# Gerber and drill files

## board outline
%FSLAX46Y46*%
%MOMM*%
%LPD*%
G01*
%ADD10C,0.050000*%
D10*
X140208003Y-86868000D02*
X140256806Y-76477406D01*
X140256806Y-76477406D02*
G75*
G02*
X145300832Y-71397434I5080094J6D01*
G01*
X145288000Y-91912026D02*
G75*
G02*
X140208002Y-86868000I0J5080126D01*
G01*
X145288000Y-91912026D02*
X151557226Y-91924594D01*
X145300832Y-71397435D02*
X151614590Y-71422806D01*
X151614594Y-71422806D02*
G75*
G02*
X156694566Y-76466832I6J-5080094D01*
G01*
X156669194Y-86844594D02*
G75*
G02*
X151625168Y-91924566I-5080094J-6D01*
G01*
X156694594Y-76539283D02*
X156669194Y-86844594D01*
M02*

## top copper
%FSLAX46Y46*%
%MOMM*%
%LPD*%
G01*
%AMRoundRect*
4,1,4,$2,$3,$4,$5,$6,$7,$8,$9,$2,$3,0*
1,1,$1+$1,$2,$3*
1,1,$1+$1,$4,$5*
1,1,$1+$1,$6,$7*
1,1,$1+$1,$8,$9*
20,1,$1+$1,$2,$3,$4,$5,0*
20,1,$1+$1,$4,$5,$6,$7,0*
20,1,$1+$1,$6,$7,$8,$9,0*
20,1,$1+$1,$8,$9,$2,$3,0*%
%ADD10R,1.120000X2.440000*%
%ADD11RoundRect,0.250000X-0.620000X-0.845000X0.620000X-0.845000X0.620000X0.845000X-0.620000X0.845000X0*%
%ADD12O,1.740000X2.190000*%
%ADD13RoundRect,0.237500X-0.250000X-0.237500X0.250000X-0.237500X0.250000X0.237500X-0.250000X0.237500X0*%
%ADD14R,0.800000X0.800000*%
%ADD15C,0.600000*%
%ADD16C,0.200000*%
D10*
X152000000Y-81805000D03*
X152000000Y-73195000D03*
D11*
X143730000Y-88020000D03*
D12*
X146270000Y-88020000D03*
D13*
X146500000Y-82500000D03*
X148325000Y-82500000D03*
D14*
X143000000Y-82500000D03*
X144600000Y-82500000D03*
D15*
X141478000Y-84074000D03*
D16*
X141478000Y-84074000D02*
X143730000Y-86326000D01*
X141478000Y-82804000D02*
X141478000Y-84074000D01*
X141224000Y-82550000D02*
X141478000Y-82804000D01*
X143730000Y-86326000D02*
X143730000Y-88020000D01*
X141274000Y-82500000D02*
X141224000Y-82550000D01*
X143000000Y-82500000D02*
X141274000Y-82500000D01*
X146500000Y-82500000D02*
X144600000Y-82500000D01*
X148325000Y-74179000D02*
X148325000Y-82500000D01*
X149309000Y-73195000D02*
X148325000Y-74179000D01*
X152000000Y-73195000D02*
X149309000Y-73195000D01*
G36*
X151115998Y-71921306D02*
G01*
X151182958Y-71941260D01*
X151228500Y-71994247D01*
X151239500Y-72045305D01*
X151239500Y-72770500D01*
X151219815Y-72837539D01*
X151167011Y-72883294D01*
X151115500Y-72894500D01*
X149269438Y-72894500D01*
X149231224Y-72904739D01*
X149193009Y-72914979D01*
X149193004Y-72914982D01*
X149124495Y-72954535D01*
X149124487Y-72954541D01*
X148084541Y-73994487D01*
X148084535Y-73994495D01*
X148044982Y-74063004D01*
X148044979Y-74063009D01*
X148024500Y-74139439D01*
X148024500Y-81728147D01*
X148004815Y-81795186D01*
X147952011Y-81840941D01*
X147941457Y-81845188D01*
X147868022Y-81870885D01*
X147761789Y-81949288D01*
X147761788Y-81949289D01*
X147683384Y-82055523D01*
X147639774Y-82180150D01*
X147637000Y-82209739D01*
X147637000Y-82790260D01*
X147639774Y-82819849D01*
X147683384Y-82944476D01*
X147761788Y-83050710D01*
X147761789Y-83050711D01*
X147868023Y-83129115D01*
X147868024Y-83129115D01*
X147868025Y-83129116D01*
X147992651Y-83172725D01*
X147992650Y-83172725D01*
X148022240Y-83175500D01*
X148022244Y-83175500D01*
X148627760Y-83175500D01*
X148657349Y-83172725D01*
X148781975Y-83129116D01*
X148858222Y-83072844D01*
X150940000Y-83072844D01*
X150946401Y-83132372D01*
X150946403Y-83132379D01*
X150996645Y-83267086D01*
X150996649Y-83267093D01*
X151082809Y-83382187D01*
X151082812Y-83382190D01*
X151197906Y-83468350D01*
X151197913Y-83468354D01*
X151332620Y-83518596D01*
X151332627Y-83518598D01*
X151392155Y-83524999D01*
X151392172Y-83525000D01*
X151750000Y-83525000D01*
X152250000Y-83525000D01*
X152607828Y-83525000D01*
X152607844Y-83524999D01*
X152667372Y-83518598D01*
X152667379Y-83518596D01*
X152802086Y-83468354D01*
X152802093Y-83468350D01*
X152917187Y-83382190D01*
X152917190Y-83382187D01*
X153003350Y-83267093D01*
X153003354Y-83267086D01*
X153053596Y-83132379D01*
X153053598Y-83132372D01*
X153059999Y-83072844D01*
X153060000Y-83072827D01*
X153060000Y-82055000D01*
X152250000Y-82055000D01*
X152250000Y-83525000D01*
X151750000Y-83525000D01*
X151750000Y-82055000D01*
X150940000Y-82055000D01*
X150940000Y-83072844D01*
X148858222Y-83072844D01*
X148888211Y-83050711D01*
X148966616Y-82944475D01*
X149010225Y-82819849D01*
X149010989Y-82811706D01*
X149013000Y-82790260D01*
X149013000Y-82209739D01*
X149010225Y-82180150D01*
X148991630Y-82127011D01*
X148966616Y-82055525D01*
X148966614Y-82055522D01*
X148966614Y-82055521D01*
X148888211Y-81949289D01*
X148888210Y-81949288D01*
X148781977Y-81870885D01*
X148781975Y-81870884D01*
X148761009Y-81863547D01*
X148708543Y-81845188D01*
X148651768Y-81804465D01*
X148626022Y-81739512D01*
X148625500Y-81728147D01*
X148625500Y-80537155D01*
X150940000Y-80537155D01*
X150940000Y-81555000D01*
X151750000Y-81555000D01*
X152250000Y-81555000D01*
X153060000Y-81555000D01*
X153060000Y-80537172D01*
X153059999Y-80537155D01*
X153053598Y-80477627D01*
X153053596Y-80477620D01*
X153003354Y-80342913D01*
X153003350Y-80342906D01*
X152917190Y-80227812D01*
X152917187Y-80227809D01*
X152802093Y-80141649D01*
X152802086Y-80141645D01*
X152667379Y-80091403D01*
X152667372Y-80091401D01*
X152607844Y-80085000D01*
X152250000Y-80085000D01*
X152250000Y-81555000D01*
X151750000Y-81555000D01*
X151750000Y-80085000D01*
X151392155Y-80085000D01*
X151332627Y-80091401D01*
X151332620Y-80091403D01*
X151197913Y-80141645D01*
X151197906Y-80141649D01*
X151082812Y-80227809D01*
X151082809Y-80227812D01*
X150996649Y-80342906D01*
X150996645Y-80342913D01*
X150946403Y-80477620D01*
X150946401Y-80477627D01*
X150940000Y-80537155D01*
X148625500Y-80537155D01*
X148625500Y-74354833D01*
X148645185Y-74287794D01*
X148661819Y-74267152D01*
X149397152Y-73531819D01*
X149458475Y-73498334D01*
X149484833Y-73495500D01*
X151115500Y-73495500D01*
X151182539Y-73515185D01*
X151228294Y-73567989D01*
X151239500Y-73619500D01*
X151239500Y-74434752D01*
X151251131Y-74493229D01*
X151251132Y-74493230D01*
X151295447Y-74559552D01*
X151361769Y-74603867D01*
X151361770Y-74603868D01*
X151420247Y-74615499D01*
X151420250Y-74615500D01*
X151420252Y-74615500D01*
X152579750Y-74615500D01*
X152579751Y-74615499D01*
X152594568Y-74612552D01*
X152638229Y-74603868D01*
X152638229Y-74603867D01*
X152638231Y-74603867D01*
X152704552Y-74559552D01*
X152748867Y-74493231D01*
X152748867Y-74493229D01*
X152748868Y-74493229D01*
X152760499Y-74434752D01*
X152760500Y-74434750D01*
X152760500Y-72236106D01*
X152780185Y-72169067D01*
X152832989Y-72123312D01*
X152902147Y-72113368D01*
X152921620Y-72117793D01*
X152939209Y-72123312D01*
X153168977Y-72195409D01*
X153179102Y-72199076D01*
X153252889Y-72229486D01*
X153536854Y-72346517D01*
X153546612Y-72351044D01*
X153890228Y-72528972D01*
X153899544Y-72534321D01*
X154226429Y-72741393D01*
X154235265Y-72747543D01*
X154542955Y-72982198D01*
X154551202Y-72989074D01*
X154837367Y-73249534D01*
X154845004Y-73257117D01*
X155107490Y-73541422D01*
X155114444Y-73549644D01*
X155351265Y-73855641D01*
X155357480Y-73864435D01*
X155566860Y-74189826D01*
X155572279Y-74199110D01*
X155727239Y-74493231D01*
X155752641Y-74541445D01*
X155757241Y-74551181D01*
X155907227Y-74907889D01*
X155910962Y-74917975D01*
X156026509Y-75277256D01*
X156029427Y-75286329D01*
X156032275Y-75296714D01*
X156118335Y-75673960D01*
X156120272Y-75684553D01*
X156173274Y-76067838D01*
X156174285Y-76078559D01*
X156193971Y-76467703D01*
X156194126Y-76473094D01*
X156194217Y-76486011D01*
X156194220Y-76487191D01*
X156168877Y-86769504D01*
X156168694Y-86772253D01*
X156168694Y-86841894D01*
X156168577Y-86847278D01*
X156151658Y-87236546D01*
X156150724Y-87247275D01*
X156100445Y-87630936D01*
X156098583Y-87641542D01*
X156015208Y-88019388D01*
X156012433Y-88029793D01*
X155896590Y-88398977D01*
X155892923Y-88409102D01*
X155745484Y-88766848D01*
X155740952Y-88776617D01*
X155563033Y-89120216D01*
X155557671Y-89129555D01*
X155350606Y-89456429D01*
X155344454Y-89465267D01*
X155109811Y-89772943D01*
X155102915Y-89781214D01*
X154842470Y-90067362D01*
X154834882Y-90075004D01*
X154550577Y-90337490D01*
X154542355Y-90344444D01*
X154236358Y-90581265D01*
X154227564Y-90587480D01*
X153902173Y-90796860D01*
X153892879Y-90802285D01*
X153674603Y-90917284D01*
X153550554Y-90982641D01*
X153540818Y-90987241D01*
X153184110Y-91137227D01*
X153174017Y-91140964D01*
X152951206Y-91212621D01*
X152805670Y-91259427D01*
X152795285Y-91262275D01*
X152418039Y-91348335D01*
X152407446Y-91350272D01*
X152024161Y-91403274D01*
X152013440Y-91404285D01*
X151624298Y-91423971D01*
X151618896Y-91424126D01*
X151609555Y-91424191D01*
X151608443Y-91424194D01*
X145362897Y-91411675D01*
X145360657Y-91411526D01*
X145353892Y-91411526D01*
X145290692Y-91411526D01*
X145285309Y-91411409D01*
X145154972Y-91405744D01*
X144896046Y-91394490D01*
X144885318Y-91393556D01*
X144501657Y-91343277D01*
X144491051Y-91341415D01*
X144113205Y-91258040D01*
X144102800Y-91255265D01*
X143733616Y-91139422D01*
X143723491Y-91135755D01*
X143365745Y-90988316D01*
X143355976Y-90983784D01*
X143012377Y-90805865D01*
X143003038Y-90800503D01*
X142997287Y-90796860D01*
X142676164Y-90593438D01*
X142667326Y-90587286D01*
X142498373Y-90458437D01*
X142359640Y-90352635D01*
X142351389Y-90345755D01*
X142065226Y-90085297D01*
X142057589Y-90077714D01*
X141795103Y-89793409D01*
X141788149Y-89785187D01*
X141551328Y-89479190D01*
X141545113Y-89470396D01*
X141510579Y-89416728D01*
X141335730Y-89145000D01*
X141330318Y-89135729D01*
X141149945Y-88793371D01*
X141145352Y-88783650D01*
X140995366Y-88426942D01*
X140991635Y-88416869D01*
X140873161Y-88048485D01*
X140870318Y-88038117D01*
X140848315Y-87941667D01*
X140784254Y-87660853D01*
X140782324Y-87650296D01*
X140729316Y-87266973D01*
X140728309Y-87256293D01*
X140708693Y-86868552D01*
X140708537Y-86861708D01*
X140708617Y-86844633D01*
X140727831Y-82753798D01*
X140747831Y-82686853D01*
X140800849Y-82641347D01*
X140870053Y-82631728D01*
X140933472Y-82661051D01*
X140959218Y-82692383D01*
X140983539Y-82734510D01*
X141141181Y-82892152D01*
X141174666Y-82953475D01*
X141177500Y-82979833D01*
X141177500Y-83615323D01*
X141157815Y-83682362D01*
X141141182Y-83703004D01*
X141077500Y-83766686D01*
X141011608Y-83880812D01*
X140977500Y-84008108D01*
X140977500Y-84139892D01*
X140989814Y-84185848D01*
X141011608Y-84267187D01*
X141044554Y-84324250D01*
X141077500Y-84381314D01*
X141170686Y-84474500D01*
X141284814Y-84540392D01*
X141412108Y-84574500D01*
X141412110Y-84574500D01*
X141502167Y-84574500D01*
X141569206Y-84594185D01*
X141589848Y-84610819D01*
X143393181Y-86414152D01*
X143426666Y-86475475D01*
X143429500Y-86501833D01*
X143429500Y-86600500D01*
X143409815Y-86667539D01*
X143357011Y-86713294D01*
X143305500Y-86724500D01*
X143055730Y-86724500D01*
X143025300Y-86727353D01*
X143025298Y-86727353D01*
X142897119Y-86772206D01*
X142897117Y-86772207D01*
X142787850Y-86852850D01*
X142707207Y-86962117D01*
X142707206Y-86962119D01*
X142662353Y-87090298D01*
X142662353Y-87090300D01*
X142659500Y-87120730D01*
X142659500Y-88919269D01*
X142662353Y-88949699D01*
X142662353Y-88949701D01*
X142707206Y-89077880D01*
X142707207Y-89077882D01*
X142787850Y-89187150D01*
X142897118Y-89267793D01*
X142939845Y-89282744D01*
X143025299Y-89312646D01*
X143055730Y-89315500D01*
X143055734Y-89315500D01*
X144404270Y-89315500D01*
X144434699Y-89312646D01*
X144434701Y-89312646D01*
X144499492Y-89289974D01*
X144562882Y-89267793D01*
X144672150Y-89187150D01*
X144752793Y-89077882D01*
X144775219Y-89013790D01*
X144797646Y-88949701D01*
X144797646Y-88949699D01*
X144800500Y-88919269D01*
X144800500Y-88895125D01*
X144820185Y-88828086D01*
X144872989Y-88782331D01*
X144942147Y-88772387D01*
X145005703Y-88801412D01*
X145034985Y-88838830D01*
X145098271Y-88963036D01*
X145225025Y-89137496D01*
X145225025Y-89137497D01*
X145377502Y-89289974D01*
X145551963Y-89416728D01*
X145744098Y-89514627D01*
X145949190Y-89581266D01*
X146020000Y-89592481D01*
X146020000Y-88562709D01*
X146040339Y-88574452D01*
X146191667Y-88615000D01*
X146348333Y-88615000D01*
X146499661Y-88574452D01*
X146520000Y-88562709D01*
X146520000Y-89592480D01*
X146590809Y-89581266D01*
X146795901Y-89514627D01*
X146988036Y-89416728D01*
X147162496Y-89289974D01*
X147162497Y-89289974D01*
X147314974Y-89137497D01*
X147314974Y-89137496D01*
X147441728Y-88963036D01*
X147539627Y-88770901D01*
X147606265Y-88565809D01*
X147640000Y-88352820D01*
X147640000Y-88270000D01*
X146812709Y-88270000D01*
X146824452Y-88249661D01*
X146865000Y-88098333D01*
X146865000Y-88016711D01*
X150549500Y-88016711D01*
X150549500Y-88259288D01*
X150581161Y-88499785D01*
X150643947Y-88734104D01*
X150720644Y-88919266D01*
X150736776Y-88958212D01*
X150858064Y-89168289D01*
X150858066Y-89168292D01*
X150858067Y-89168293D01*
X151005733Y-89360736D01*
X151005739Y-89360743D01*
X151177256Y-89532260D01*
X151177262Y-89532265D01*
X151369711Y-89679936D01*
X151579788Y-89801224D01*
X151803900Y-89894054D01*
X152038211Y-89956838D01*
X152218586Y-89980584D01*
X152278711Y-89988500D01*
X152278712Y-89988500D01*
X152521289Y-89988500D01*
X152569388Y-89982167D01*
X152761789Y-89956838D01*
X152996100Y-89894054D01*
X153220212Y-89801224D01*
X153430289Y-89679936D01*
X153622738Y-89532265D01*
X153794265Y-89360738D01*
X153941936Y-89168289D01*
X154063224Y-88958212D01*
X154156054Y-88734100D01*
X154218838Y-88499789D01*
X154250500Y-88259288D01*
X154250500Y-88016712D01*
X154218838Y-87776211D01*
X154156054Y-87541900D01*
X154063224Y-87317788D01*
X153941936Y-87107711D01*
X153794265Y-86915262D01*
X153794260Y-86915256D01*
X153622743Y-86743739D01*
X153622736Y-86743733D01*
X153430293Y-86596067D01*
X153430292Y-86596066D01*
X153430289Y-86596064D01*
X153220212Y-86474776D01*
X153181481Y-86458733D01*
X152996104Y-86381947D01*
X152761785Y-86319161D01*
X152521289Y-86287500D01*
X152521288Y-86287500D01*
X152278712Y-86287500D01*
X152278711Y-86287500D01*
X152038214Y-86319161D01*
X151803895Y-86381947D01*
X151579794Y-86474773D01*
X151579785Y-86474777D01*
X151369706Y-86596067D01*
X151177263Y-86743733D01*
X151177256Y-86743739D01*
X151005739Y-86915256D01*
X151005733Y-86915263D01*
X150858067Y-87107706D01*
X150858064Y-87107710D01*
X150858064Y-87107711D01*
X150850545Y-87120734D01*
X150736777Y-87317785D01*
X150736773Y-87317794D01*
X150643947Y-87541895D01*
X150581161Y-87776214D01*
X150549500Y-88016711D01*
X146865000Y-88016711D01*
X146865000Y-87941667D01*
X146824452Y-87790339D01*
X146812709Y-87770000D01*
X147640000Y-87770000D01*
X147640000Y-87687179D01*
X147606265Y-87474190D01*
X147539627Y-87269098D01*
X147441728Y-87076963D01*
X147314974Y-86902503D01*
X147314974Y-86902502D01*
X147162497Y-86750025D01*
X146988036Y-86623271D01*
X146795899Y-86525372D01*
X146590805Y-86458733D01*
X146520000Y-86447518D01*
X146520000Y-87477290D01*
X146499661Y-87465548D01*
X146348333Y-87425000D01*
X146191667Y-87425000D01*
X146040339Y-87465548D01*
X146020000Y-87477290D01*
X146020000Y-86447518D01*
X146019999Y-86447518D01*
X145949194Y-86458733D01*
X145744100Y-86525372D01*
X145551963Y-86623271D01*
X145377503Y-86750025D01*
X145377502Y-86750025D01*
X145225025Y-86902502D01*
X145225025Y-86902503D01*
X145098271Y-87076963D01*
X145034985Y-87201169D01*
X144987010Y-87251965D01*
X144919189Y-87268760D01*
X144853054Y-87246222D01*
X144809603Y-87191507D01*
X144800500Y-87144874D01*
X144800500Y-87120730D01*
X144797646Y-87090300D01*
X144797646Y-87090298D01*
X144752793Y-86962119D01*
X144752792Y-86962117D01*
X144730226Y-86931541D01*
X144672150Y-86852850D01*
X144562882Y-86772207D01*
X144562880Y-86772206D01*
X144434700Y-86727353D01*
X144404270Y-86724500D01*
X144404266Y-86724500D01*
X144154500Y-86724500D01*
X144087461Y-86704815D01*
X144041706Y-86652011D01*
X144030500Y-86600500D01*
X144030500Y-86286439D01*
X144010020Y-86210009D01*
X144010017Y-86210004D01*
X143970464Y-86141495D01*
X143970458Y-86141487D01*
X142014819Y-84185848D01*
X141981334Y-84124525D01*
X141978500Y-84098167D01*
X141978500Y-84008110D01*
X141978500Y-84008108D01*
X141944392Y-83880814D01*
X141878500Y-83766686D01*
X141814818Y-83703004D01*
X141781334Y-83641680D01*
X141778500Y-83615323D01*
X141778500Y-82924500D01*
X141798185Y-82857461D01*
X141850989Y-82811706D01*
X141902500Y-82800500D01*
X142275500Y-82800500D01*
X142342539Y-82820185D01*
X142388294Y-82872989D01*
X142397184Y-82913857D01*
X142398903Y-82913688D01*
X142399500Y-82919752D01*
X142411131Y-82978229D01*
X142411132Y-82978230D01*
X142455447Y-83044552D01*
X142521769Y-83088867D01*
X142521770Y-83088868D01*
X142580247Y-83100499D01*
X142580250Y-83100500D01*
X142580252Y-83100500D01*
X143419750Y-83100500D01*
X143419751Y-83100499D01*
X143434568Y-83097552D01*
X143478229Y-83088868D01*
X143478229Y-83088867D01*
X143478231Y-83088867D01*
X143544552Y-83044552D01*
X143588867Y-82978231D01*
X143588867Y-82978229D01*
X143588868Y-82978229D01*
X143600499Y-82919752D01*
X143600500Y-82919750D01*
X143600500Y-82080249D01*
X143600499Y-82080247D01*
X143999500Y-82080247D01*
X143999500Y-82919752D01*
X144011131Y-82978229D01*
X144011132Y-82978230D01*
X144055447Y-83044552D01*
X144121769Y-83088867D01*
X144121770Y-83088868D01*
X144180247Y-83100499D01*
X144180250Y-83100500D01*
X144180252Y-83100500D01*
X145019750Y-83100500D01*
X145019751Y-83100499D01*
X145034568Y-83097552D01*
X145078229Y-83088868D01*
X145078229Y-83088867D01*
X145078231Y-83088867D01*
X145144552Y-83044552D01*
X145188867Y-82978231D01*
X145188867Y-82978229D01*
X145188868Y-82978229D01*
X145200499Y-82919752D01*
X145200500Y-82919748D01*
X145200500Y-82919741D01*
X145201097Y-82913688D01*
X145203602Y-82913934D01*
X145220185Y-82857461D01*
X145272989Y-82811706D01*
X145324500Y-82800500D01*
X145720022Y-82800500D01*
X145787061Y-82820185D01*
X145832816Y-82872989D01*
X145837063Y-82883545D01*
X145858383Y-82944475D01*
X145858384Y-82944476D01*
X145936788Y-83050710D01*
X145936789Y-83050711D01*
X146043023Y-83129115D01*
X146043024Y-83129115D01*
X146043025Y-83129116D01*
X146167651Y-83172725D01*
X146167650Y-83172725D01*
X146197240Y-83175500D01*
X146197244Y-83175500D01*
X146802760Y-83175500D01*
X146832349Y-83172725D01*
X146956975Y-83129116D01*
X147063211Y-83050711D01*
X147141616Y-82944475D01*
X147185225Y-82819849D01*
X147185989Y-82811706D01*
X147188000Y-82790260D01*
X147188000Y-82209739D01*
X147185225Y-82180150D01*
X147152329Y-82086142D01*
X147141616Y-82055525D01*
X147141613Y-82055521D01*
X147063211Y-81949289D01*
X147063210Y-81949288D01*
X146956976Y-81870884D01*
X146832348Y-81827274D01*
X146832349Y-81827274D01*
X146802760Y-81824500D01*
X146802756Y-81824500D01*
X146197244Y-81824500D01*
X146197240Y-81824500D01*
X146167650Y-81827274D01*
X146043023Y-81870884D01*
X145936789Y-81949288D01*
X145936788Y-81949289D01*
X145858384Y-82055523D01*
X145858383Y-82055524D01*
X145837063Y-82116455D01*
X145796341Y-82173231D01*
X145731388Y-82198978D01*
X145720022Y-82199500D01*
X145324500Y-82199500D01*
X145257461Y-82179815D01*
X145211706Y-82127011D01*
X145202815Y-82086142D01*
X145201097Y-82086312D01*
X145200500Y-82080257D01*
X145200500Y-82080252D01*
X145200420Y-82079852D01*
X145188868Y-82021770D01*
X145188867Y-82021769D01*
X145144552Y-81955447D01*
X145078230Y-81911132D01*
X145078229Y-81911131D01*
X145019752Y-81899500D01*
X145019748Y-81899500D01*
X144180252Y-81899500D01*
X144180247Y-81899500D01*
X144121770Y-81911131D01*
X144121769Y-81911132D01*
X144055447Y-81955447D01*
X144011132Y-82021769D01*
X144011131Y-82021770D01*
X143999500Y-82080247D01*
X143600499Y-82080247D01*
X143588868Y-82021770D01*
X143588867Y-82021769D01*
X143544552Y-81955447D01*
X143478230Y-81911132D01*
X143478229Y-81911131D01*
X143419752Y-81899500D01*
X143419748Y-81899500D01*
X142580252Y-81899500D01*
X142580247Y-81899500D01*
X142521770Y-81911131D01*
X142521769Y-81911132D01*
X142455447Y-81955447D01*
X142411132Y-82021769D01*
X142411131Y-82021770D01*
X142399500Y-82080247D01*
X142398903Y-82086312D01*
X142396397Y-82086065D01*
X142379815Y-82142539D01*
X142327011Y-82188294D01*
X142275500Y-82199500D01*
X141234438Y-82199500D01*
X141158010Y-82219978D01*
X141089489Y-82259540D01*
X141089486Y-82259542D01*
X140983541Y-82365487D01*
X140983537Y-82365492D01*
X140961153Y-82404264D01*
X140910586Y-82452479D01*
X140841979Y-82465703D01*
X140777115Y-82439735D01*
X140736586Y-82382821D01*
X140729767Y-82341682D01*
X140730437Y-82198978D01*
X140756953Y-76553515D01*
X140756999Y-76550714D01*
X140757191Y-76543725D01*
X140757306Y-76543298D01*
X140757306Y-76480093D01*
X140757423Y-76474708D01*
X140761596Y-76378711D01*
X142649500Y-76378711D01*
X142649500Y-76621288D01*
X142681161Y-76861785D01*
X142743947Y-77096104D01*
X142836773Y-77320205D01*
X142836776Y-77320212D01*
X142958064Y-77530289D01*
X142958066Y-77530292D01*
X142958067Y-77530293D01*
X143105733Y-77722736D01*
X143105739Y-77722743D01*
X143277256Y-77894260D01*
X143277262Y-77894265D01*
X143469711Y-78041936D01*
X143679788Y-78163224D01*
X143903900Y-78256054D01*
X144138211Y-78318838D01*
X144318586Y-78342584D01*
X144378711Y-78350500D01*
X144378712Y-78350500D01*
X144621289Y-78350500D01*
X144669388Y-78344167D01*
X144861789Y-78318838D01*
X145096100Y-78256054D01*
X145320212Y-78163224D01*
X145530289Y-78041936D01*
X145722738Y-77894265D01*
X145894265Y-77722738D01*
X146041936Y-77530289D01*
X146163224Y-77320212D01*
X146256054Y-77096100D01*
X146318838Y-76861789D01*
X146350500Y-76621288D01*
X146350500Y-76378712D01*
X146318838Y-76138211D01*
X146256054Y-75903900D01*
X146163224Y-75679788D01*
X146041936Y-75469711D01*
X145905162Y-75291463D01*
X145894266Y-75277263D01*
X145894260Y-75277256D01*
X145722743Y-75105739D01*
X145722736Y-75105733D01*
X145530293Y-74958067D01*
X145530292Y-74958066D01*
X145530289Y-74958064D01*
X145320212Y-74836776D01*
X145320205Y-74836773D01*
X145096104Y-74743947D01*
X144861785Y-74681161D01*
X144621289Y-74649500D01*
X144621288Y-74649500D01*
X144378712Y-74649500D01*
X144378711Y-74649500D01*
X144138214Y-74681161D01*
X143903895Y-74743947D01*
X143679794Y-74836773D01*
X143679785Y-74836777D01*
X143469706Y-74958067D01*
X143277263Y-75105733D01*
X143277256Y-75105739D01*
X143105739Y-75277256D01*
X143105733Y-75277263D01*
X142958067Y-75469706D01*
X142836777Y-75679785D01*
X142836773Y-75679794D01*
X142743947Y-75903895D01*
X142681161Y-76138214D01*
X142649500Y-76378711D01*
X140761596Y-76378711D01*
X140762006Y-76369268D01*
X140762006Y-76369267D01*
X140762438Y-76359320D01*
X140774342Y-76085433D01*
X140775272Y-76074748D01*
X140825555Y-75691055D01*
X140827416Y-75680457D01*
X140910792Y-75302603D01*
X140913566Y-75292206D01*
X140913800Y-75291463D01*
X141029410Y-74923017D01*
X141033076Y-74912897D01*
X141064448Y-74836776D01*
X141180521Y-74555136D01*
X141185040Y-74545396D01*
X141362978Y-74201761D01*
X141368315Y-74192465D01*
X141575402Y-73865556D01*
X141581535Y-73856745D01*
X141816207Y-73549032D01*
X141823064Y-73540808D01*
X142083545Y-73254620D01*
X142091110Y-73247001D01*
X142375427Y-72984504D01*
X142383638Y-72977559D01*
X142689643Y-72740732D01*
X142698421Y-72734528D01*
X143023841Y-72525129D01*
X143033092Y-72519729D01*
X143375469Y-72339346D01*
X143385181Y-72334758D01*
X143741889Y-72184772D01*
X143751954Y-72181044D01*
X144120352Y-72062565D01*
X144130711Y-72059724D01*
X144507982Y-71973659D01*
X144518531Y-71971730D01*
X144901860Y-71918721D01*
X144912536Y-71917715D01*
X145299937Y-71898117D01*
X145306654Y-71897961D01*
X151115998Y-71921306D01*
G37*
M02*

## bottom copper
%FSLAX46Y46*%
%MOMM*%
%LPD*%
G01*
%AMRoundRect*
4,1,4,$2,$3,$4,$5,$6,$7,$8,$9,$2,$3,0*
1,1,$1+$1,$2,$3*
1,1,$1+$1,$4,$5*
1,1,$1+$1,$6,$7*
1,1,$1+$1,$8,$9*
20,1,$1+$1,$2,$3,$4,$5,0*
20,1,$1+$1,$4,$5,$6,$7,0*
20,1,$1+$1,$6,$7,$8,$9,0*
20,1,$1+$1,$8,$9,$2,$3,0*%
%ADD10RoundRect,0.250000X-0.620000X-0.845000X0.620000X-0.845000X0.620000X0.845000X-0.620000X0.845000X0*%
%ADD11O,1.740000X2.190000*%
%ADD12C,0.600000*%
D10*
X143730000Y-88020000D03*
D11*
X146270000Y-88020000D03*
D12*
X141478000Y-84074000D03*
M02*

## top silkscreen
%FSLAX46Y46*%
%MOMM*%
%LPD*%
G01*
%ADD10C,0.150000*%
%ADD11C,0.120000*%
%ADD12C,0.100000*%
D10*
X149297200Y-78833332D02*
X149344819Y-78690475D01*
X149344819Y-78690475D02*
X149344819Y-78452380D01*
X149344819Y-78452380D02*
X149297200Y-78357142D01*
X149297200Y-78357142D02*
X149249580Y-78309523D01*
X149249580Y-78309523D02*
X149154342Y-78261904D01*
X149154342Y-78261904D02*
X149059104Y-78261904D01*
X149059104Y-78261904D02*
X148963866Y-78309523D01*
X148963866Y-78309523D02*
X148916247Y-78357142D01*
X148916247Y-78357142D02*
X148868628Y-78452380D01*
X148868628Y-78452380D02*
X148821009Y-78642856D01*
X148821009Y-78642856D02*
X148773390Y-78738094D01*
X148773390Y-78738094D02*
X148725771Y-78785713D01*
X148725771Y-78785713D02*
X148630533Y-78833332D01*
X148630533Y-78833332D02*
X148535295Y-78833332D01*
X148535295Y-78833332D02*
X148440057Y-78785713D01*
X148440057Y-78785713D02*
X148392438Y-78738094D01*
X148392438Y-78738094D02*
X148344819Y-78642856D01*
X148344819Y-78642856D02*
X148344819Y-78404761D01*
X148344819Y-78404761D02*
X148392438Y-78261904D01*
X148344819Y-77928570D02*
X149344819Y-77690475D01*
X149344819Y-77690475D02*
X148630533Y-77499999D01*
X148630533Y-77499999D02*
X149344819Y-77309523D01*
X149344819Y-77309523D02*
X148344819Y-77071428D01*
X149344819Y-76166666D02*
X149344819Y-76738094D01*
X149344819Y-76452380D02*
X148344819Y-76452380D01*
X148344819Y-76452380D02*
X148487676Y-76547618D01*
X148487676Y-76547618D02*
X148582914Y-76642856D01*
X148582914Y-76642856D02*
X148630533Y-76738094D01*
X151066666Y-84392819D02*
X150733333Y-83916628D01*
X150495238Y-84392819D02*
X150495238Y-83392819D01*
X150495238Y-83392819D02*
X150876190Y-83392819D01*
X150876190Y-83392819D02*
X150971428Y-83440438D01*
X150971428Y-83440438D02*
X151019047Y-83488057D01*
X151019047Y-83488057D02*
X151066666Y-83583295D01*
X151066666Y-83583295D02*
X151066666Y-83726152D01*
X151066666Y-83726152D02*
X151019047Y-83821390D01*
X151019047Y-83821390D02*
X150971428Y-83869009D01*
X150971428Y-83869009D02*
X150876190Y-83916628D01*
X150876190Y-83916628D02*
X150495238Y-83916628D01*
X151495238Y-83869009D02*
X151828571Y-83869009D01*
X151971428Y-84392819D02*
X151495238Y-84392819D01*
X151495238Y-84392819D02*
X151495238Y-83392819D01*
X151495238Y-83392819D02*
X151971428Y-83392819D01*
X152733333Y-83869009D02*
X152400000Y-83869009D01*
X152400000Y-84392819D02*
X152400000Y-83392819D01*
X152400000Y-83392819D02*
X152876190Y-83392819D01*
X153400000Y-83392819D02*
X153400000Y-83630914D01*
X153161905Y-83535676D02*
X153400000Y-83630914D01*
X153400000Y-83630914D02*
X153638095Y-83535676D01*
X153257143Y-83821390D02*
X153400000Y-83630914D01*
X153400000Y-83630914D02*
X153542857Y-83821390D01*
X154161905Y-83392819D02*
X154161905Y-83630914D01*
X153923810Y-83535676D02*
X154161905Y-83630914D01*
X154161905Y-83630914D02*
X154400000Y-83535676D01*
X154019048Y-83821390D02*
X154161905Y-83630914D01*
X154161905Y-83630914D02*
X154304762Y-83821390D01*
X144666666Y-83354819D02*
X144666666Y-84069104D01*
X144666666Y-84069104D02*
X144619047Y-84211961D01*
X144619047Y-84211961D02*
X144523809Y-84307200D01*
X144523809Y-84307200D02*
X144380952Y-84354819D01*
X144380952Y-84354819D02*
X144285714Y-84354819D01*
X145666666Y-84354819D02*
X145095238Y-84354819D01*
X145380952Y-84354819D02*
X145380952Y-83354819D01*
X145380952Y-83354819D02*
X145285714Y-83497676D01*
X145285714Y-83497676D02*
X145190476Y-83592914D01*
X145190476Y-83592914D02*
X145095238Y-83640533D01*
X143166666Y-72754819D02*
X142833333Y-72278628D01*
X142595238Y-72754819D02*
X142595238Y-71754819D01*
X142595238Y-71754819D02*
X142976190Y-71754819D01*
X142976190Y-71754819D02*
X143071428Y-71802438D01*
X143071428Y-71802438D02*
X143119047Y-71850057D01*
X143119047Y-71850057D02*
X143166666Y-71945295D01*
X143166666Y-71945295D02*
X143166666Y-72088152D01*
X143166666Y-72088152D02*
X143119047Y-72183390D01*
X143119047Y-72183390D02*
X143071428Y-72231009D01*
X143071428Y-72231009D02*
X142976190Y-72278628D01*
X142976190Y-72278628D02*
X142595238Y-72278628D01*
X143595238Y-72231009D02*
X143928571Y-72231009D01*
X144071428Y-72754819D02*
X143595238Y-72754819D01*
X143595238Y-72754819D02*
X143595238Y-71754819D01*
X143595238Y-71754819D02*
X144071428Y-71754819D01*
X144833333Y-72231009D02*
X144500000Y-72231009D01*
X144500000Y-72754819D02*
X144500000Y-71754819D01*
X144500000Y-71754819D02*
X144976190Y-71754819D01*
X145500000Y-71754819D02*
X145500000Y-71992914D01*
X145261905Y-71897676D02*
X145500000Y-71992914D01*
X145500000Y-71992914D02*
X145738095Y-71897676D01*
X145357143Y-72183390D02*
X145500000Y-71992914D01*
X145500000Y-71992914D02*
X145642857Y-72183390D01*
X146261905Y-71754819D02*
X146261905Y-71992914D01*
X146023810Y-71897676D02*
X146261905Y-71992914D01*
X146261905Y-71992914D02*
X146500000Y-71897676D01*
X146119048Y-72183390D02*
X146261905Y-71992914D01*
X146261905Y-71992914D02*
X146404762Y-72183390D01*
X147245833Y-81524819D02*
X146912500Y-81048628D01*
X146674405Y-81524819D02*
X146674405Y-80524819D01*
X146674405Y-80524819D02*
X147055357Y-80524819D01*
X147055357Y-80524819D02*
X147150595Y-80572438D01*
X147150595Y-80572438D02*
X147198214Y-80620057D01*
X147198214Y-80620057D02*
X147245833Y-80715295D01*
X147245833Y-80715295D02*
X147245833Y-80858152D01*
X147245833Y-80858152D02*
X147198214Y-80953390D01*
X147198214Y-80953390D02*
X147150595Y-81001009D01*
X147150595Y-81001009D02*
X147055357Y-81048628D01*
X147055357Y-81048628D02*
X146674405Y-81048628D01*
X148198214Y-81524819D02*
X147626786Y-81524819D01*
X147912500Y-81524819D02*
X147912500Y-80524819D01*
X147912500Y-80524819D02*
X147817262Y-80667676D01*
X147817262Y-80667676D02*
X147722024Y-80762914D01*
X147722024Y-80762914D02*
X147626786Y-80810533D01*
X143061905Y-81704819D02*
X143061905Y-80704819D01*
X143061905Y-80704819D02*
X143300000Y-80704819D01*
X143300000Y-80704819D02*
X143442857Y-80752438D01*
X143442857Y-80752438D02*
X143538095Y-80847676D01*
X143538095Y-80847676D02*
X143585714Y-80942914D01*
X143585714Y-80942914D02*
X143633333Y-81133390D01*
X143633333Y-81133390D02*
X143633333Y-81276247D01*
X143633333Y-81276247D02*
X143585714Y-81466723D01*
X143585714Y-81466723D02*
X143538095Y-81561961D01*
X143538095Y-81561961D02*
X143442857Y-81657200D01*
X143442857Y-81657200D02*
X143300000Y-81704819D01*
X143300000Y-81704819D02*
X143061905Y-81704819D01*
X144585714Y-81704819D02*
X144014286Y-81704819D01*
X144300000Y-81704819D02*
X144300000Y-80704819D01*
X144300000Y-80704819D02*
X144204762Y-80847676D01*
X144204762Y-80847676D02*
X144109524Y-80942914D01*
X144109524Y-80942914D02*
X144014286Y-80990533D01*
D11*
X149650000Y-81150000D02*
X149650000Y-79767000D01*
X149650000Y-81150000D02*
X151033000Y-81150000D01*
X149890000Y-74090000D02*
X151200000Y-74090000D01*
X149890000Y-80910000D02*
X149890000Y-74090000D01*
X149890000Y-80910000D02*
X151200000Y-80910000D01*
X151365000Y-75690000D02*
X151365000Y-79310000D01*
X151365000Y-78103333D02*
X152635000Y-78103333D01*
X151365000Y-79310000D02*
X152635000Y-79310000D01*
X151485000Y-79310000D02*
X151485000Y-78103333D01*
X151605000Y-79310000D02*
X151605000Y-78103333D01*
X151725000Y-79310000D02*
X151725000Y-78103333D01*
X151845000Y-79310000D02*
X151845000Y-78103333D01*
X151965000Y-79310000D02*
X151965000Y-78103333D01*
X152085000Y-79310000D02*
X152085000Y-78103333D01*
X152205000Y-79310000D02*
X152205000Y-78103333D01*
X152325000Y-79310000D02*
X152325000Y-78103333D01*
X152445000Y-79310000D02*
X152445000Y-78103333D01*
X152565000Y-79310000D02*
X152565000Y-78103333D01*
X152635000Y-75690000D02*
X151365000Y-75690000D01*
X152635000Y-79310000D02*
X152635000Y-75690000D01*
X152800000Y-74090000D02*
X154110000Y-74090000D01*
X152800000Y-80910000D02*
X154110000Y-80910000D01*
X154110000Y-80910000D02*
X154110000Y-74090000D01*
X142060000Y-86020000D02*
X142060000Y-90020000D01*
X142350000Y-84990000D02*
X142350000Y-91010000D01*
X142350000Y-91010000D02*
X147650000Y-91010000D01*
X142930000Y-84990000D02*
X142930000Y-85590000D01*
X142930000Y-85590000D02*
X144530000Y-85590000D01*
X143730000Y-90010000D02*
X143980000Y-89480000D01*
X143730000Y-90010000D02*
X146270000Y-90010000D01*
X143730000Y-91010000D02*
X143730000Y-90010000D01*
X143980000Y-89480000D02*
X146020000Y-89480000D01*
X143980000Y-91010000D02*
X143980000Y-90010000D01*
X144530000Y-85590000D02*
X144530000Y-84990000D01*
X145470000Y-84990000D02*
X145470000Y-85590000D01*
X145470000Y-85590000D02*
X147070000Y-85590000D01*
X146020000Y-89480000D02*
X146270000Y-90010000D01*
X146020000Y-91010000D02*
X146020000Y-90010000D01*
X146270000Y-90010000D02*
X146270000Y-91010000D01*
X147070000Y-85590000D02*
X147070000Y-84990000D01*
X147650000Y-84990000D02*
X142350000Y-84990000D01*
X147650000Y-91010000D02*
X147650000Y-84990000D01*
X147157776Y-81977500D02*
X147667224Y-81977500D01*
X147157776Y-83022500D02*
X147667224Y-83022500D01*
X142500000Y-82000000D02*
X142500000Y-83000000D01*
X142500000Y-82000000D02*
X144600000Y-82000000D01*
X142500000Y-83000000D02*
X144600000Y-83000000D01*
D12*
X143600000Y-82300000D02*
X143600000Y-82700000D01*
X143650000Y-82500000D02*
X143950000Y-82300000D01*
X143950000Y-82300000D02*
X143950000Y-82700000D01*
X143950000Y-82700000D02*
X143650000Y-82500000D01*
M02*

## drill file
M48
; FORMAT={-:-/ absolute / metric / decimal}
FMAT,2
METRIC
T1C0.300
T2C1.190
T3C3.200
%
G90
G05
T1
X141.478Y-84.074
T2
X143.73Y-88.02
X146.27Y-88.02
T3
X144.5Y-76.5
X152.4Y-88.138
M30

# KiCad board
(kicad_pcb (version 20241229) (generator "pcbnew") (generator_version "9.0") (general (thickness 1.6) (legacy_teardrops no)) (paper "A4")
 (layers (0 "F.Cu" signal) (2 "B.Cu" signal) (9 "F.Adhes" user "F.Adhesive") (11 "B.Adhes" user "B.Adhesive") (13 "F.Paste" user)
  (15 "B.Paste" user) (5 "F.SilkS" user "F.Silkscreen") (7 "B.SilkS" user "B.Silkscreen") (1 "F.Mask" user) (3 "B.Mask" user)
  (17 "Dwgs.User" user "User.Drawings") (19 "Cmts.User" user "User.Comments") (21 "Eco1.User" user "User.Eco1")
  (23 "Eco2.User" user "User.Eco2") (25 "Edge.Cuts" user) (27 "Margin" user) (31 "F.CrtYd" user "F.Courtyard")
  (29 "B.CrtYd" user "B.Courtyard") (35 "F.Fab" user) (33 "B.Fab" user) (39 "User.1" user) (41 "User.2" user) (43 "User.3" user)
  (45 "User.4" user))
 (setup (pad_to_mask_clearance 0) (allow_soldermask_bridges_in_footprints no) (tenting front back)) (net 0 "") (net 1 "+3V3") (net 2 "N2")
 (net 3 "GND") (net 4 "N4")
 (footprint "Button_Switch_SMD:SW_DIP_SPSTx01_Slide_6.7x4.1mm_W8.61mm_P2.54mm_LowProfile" (layer "F.Cu") (at 152 77.5 90)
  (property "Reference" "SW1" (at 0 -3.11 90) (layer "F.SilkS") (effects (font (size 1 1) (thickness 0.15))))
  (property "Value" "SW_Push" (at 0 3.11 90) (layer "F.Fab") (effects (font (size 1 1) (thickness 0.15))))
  (fp_line (start -3.65 -2.35) (end -2.267 -2.35) (stroke (width 0.12) (type solid)) (layer "F.SilkS"))
  (fp_line (start -3.65 -2.35) (end -3.65 -0.967) (stroke (width 0.12) (type solid)) (layer "F.SilkS"))
  (fp_line (start 3.41 -2.11) (end 3.41 -0.8) (stroke (width 0.12) (type solid)) (layer "F.SilkS"))
  (fp_line (start -3.41 -2.11) (end 3.41 -2.11) (stroke (width 0.12) (type solid)) (layer "F.SilkS"))
  (fp_line (start -3.41 -2.11) (end -3.41 -0.8) (stroke (width 0.12) (type solid)) (layer "F.SilkS"))
  (fp_line (start 1.81 -0.635) (end -1.81 -0.635) (stroke (width 0.12) (type solid)) (layer "F.SilkS"))
  (fp_line (start -0.603333 -0.635) (end -0.603333 0.635) (stroke (width 0.12) (type solid)) (layer "F.SilkS"))
  (fp_line (start -1.81 -0.635) (end -1.81 0.635) (stroke (width 0.12) (type solid)) (layer "F.SilkS"))
  (fp_line (start -1.81 -0.515) (end -0.603333 -0.515) (stroke (width 0.12) (type solid)) (layer "F.SilkS"))
  (fp_line (start -1.81 -0.395) (end -0.603333 -0.395) (stroke (width 0.12) (type solid)) (layer "F.SilkS"))
  (fp_line (start -1.81 -0.275) (end -0.603333 -0.275) (stroke (width 0.12) (type solid)) (layer "F.SilkS"))
  (fp_line (start -1.81 -0.155) (end -0.603333 -0.155) (stroke (width 0.12) (type solid)) (layer "F.SilkS"))
  (fp_line (start -1.81 -0.035) (end -0.603333 -0.035) (stroke (width 0.12) (type solid)) (layer "F.SilkS"))
  (fp_line (start -1.81 0.085) (end -0.603333 0.085) (stroke (width 0.12) (type solid)) (layer "F.SilkS"))
  (fp_line (start -1.81 0.205) (end -0.603333 0.205) (stroke (width 0.12) (type solid)) (layer "F.SilkS"))
  (fp_line (start -1.81 0.325) (end -0.603333 0.325) (stroke (width 0.12) (type solid)) (layer "F.SilkS"))
  (fp_line (start -1.81 0.445) (end -0.603333 0.445) (stroke (width 0.12) (type solid)) (layer "F.SilkS"))
  (fp_line (start -1.81 0.565) (end -0.603333 0.565) (stroke (width 0.12) (type solid)) (layer "F.SilkS"))
  (fp_line (start 1.81 0.635) (end 1.81 -0.635) (stroke (width 0.12) (type solid)) (layer "F.SilkS"))
  (fp_line (start -1.81 0.635) (end 1.81 0.635) (stroke (width 0.12) (type solid)) (layer "F.SilkS"))
  (fp_line (start 3.41 0.8) (end 3.41 2.11) (stroke (width 0.12) (type solid)) (layer "F.SilkS"))
  (fp_line (start -3.41 0.8) (end -3.41 2.11) (stroke (width 0.12) (type solid)) (layer "F.SilkS"))
  (fp_line (start -3.41 2.11) (end 3.41 2.11) (stroke (width 0.12) (type solid)) (layer "F.SilkS"))
  (pad "1" smd rect (at -4.305 0 90) (size 2.44 1.12) (layers "F.Cu" "F.Mask" "F.Paste") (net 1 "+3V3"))
  (pad "2" smd rect (at 4.305 0 90) (size 2.44 1.12) (layers "F.Cu" "F.Mask" "F.Paste") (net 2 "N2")))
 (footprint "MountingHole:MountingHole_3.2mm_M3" (layer "F.Cu") (at 152.4 88.138)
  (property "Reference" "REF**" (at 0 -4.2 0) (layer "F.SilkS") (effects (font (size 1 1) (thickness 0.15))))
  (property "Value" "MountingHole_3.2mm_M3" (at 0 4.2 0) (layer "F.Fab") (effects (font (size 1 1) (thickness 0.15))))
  (pad "" np_thru_hole circle (at 0 0) (size 3.2 3.2) (drill 3.2) (layers "*.Cu" "*.Mask")))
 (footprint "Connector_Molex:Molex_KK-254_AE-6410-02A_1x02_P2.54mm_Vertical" (layer "F.Cu") (at 143.73 88.02)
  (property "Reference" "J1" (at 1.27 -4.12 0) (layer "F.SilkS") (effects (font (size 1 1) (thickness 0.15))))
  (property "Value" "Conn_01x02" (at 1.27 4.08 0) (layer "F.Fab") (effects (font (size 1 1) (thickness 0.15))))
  (fp_line (start -1.67 -2) (end -1.67 2) (stroke (width 0.12) (type solid)) (layer "F.SilkS"))
  (fp_line (start -1.38 -3.03) (end -1.38 2.99) (stroke (width 0.12) (type solid)) (layer "F.SilkS"))
  (fp_line (start -1.38 2.99) (end 3.92 2.99) (stroke (width 0.12) (type solid)) (layer "F.SilkS"))
  (fp_line (start -0.8 -3.03) (end -0.8 -2.43) (stroke (width 0.12) (type solid)) (layer "F.SilkS"))
  (fp_line (start -0.8 -2.43) (end 0.8 -2.43) (stroke (width 0.12) (type solid)) (layer "F.SilkS"))
  (fp_line (start 0 1.99) (end 0.25 1.46) (stroke (width 0.12) (type solid)) (layer "F.SilkS"))
  (fp_line (start 0 1.99) (end 2.54 1.99) (stroke (width 0.12) (type solid)) (layer "F.SilkS"))
  (fp_line (start 0 2.99) (end 0 1.99) (stroke (width 0.12) (type solid)) (layer "F.SilkS"))
  (fp_line (start 0.25 1.46) (end 2.29 1.46) (stroke (width 0.12) (type solid)) (layer "F.SilkS"))
  (fp_line (start 0.25 2.99) (end 0.25 1.99) (stroke (width 0.12) (type solid)) (layer "F.SilkS"))
  (fp_line (start 0.8 -2.43) (end 0.8 -3.03) (stroke (width 0.12) (type solid)) (layer "F.SilkS"))
  (fp_line (start 1.74 -3.03) (end 1.74 -2.43) (stroke (width 0.12) (type solid)) (layer "F.SilkS"))
  (fp_line (start 1.74 -2.43) (end 3.34 -2.43) (stroke (width 0.12) (type solid)) (layer "F.SilkS"))
  (fp_line (start 2.29 1.46) (end 2.54 1.99) (stroke (width 0.12) (type solid)) (layer "F.SilkS"))
  (fp_line (start 2.29 2.99) (end 2.29 1.99) (stroke (width 0.12) (type solid)) (layer "F.SilkS"))
  (fp_line (start 2.54 1.99) (end 2.54 2.99) (stroke (width 0.12) (type solid)) (layer "F.SilkS"))
  (fp_line (start 3.34 -2.43) (end 3.34 -3.03) (stroke (width 0.12) (type solid)) (layer "F.SilkS"))
  (fp_line (start 3.92 -3.03) (end -1.38 -3.03) (stroke (width 0.12) (type solid)) (layer "F.SilkS"))
  (fp_line (start 3.92 2.99) (end 3.92 -3.03) (stroke (width 0.12) (type solid)) (layer "F.SilkS"))
  (pad "1" thru_hole roundrect (at 0 0) (size 1.74 2.19) (drill 1.19) (layers "*.Cu" "*.Mask") (remove_unused_layers no)
   (roundrect_rratio 0.143678) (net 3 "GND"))
  (pad "2" thru_hole oval (at 2.54 0) (size 1.74 2.19) (drill 1.19) (layers "*.Cu" "*.Mask") (remove_unused_layers no) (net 1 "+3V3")))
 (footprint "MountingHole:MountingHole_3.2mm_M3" (layer "F.Cu") (at 144.5 76.5)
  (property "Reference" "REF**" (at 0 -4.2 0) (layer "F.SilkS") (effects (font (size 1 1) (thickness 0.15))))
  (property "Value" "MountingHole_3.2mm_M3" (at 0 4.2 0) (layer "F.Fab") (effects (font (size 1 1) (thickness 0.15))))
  (pad "" np_thru_hole circle (at 0 0) (size 3.2 3.2) (drill 3.2) (layers "*.Cu" "*.Mask")))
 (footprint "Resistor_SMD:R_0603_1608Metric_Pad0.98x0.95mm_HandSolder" (layer "F.Cu") (at 147.4125 82.5)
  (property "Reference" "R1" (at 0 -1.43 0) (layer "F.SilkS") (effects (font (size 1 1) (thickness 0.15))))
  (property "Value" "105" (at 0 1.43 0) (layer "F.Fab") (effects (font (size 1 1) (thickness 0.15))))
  (fp_line (start -0.254724 -0.5225) (end 0.254724 -0.5225) (stroke (width 0.12) (type solid)) (layer "F.SilkS"))
  (fp_line (start -0.254724 0.5225) (end 0.254724 0.5225) (stroke (width 0.12) (type solid)) (layer "F.SilkS"))
  (pad "1" smd roundrect (at -0.9125 0) (size 0.975 0.95) (layers "F.Cu" "F.Mask" "F.Paste") (roundrect_rratio 0.25) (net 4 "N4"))
  (pad "2" smd roundrect (at 0.9125 0) (size 0.975 0.95) (layers "F.Cu" "F.Mask" "F.Paste") (roundrect_rratio 0.25) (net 2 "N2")))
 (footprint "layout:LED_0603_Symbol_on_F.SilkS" (layer "F.Cu") (at 143.8 82.5)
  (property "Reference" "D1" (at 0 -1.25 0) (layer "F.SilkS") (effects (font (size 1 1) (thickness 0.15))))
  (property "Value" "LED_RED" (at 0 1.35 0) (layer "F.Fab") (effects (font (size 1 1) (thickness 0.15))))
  (fp_line (start -1.3 -0.5) (end -1.3 0.5) (stroke (width 0.12) (type solid)) (layer "F.SilkS"))
  (fp_line (start -1.3 -0.5) (end 0.8 -0.5) (stroke (width 0.12) (type solid)) (layer "F.SilkS"))
  (fp_line (start -1.3 0.5) (end 0.8 0.5) (stroke (width 0.12) (type solid)) (layer "F.SilkS"))
  (fp_line (start -0.2 -0.2) (end -0.2 0.2) (stroke (width 0.1) (type solid)) (layer "F.SilkS"))
  (fp_line (start -0.15 0) (end 0.15 -0.2) (stroke (width 0.1) (type solid)) (layer "F.SilkS"))
  (fp_line (start 0.15 -0.2) (end 0.15 0.2) (stroke (width 0.1) (type solid)) (layer "F.SilkS"))
  (fp_line (start 0.15 0.2) (end -0.15 0) (stroke (width 0.1) (type solid)) (layer "F.SilkS"))
  (pad "1" smd rect (at -0.8 0 180) (size 0.8 0.8) (layers "F.Cu" "F.Mask" "F.Paste") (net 3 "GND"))
  (pad "2" smd rect (at 0.8 0 180) (size 0.8 0.8) (layers "F.Cu" "F.Mask" "F.Paste") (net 4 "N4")))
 (gr_line (start 140.208003 86.868) (end 140.256806 76.477406) (stroke (width 0.05) (type default)) (layer "Edge.Cuts"))
 (gr_arc (start 140.256806 76.477406) (mid 141.732 72.898) (end 145.300832 71.397406) (stroke (width 0.05) (type default))
  (layer "Edge.Cuts"))
 (gr_arc (start 145.288 91.912026) (mid 141.708594 90.436832) (end 140.208 86.868) (stroke (width 0.05) (type default)) (layer "Edge.Cuts"))
 (gr_line (start 145.288 91.912026) (end 151.557226 91.924594) (stroke (width 0.05) (type default)) (layer "Edge.Cuts"))
 (gr_line (start 145.300832 71.397435) (end 151.61459 71.422806) (stroke (width 0.05) (type default)) (layer "Edge.Cuts"))
 (gr_arc (start 151.614594 71.422806) (mid 155.194 72.898) (end 156.694594 76.466832) (stroke (width 0.05) (type default))
  (layer "Edge.Cuts"))
 (gr_arc (start 156.669194 86.844594) (mid 155.194 90.424) (end 151.625168 91.924594) (stroke (width 0.05) (type default))
  (layer "Edge.Cuts"))
 (gr_line (start 156.694594 76.539283) (end 156.669194 86.844594) (stroke (width 0.05) (type default)) (layer "Edge.Cuts"))
 (segment (start 141.478 84.074) (end 143.73 86.326) (width 0.2) (layer "F.Cu") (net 3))
 (segment (start 141.478 82.804) (end 141.478 84.074) (width 0.2) (layer "F.Cu") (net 3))
 (segment (start 141.224 82.55) (end 141.478 82.804) (width 0.2) (layer "F.Cu") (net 3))
 (segment (start 143.73 86.326) (end 143.73 88.02) (width 0.2) (layer "F.Cu") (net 3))
 (segment (start 141.274 82.5) (end 141.224 82.55) (width 0.2) (layer "F.Cu") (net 3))
 (segment (start 143 82.5) (end 141.274 82.5) (width 0.2) (layer "F.Cu") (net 3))
 (via (at 141.478 84.074) (size 0.6) (drill 0.3) (layers "F.Cu" "B.Cu") (free yes) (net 3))
 (segment (start 146.5 82.5) (end 144.6 82.5) (width 0.2) (layer "F.Cu") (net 4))
 (segment (start 148.325 74.179) (end 148.325 82.5) (width 0.2) (layer "F.Cu") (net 2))
 (segment (start 149.309 73.195) (end 148.325 74.179) (width 0.2) (layer "F.Cu") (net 2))
 (segment (start 152 73.195) (end 149.309 73.195) (width 0.2) (layer "F.Cu") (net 2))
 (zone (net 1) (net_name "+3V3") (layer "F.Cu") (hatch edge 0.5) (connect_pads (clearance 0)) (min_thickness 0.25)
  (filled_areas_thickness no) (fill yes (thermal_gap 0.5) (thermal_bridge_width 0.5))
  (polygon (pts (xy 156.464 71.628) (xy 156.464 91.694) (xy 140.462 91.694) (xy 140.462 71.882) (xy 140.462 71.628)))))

